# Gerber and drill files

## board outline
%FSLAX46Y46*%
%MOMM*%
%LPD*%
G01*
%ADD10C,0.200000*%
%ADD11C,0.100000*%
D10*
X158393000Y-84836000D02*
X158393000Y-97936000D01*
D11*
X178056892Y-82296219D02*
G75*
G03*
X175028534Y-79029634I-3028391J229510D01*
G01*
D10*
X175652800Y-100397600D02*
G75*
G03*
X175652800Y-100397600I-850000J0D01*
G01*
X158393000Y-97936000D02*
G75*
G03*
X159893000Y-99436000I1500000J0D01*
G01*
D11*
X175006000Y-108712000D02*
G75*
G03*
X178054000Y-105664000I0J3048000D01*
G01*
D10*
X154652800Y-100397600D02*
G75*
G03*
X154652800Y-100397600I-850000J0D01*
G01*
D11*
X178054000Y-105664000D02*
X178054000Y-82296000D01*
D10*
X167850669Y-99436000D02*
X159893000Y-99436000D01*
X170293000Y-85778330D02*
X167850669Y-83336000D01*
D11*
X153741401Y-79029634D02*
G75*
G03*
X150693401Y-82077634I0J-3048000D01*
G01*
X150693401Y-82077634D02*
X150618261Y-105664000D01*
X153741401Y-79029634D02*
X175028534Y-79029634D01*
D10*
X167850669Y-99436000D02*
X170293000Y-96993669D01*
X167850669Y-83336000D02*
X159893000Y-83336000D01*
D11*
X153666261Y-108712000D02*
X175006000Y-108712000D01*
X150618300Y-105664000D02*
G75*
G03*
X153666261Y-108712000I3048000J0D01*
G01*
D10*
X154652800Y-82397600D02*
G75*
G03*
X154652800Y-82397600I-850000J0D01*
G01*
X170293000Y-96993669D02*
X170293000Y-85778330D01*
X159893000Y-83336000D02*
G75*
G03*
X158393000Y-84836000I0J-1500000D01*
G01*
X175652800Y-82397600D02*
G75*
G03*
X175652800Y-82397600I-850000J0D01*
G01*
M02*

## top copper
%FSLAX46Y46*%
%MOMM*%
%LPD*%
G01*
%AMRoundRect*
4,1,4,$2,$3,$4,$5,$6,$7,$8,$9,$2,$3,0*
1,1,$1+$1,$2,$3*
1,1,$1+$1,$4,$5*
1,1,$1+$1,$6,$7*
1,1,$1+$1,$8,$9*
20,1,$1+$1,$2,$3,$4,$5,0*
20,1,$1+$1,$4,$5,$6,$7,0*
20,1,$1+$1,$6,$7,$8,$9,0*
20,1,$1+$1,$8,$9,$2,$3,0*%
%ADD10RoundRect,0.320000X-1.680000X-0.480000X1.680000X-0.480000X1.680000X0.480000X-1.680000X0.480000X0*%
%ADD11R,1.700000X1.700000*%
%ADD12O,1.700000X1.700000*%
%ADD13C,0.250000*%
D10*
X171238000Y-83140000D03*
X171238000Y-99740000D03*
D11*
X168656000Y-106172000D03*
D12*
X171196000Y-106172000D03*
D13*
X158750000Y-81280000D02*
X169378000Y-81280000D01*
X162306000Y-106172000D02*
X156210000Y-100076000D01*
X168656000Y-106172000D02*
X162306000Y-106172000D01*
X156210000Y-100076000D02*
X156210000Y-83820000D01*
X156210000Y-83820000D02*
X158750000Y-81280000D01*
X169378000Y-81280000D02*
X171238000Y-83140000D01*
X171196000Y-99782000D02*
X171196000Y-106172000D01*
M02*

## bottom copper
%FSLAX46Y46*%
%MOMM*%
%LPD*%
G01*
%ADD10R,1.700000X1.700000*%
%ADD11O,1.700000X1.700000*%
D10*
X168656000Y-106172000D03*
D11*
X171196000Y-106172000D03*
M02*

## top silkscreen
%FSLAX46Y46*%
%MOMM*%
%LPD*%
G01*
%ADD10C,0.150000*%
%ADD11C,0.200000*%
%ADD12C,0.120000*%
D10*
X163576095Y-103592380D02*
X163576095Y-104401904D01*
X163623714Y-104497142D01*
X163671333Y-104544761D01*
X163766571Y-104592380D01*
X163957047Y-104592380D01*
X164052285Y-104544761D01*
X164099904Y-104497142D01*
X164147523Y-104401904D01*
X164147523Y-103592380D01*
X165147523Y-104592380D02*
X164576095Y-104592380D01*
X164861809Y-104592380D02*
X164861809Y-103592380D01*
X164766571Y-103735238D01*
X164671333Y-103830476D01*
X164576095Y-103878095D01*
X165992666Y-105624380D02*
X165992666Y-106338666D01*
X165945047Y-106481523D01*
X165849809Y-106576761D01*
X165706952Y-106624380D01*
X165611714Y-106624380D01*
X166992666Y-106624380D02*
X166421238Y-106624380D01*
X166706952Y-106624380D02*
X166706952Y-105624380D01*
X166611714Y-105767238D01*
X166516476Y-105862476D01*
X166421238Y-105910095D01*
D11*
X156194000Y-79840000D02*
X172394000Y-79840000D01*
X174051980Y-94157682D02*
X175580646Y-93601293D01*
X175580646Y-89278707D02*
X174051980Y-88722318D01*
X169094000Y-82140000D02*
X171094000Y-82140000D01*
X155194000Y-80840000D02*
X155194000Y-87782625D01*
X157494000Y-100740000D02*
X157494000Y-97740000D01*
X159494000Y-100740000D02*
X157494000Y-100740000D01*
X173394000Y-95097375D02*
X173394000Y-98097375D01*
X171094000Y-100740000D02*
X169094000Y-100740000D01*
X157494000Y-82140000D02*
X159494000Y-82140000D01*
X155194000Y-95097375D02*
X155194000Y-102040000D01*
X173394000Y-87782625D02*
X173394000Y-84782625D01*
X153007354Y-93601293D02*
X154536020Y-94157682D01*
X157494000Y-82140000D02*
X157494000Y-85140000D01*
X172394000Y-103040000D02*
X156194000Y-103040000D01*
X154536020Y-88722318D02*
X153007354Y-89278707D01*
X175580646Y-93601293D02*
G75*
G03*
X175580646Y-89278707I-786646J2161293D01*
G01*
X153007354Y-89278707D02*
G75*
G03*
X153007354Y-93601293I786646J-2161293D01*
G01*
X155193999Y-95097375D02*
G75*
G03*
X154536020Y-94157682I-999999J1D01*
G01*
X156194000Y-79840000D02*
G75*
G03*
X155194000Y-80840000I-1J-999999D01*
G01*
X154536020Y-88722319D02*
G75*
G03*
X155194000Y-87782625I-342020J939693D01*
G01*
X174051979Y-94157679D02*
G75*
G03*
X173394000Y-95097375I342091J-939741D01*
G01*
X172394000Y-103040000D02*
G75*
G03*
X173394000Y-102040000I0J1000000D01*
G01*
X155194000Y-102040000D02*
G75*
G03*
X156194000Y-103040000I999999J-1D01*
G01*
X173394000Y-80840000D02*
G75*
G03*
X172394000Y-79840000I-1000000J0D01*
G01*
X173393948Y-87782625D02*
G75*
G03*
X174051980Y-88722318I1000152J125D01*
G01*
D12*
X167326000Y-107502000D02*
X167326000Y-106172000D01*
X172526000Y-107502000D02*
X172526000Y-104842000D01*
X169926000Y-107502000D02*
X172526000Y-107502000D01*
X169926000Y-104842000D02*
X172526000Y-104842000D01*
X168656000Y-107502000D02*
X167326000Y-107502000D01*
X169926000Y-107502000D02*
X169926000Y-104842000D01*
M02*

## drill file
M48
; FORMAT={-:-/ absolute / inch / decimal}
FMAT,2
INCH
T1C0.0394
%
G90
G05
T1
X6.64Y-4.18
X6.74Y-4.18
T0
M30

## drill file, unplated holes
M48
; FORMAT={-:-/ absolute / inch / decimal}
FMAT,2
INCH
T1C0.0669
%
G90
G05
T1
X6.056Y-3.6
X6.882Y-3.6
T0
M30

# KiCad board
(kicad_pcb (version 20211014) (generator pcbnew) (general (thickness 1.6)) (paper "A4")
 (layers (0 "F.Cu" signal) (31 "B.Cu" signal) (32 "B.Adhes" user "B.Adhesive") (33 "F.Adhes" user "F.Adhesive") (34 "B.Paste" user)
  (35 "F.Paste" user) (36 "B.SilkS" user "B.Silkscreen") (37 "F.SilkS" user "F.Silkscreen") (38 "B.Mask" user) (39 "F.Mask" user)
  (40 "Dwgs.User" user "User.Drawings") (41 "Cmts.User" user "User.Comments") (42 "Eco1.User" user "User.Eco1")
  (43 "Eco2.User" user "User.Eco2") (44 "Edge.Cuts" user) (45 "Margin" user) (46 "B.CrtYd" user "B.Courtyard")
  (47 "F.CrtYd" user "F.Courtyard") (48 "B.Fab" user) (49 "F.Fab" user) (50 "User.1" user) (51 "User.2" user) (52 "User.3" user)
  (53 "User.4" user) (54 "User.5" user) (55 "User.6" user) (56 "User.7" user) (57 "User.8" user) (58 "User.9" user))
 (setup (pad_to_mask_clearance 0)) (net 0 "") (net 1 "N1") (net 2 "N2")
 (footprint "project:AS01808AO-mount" (layer "F.Cu") (at 164.338 91.44)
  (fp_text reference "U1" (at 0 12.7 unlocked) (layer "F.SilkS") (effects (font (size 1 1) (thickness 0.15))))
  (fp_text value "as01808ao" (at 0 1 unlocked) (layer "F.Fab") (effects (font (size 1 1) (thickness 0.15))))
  (fp_line (start -8.144 -11.6) (end 8.056 -11.6) (layer "F.SilkS") (width 0.2))
  (fp_line (start 9.71398 2.717682) (end 11.242646 2.161293) (layer "F.SilkS") (width 0.2))
  (fp_line (start 11.242646 -2.161293) (end 9.71398 -2.717682) (layer "F.SilkS") (width 0.2))
  (fp_line (start 4.756 -9.3) (end 6.756 -9.3) (layer "F.SilkS") (width 0.2))
  (fp_line (start -9.144 -10.6) (end -9.144 -3.657375) (layer "F.SilkS") (width 0.2))
  (fp_line (start -6.844 9.3) (end -6.844 6.3) (layer "F.SilkS") (width 0.2))
  (fp_line (start -4.844 9.3) (end -6.844 9.3) (layer "F.SilkS") (width 0.2))
  (fp_line (start 9.056 3.657375) (end 9.056 6.657375) (layer "F.SilkS") (width 0.2))
  (fp_line (start 6.756 9.3) (end 4.756 9.3) (layer "F.SilkS") (width 0.2))
  (fp_line (start -6.844 -9.3) (end -4.844 -9.3) (layer "F.SilkS") (width 0.2))
  (fp_line (start -9.144 3.657375) (end -9.144 10.6) (layer "F.SilkS") (width 0.2))
  (fp_line (start 9.056 -3.657375) (end 9.056 -6.657375) (layer "F.SilkS") (width 0.2))
  (fp_line (start -11.330646 2.161293) (end -9.80198 2.717682) (layer "F.SilkS") (width 0.2))
  (fp_line (start -6.844 -9.3) (end -6.844 -6.3) (layer "F.SilkS") (width 0.2))
  (fp_line (start 8.056 11.6) (end -8.144 11.6) (layer "F.SilkS") (width 0.2))
  (fp_line (start -9.80198 -2.717682) (end -11.330646 -2.161293) (layer "F.SilkS") (width 0.2))
  (fp_arc (start 11.242646 -2.161293) (mid 12.756 0) (end 11.242646 2.161293) (layer "F.SilkS") (width 0.2))
  (fp_arc (start -11.330646 2.161293) (mid -12.844 0) (end -11.330646 -2.161293) (layer "F.SilkS") (width 0.2))
  (fp_arc (start -9.80198 2.717682) (mid -9.324848 3.083798) (end -9.144 3.657375) (layer "F.SilkS") (width 0.2))
  (fp_arc (start -9.144 -10.6) (mid -8.851107 -11.307107) (end -8.144 -11.6) (layer "F.SilkS") (width 0.2))
  (fp_arc (start -9.144 -3.657375) (mid -9.324848 -3.083798) (end -9.80198 -2.717682) (layer "F.SilkS") (width 0.2))
  (fp_arc (start 9.056 3.657375) (mid 9.236859 3.083806) (end 9.71398 2.717682) (layer "F.SilkS") (width 0.2))
  (fp_arc (start 9.056 10.6) (mid 8.763107 11.307107) (end 8.056 11.6) (layer "F.SilkS") (width 0.2))
  (fp_arc (start -8.144 11.6) (mid -8.851107 11.307107) (end -9.144 10.6) (layer "F.SilkS") (width 0.2))
  (fp_arc (start 8.056 -11.6) (mid 8.763107 -11.307107) (end 9.056 -10.6) (layer "F.SilkS") (width 0.2))
  (fp_arc (start 9.71398 -2.717682) (mid 9.236845 -3.083806) (end 9.056 -3.657375) (layer "F.SilkS") (width 0.2))
  (pad "" np_thru_hole circle (at 10.4648 0) (size 1.7 1.7) (drill 1.7) (layers F&B.Cu *.Mask))
  (pad "" np_thru_hole circle (at -10.5156 0) (size 1.7 1.7) (drill 1.7) (layers F&B.Cu *.Mask))
  (pad "1" smd roundrect (at 6.9 -8.3) (size 4 1.6) (layers "F.Cu" "F.Paste" "F.Mask") (roundrect_rratio 0.2) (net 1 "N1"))
  (pad "2" smd roundrect (at 6.9 8.3) (size 4 1.6) (layers "F.Cu" "F.Paste" "F.Mask") (roundrect_rratio 0.2) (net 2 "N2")))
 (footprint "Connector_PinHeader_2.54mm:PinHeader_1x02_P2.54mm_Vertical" (layer "F.Cu") (at 168.656 106.172 90)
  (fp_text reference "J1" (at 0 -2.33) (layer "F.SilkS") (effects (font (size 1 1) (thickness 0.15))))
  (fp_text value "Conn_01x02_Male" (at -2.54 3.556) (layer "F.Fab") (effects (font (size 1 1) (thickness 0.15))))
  (fp_line (start -1.33 -1.33) (end 0 -1.33) (layer "F.SilkS") (width 0.12))
  (fp_line (start -1.33 3.87) (end 1.33 3.87) (layer "F.SilkS") (width 0.12))
  (fp_line (start -1.33 1.27) (end -1.33 3.87) (layer "F.SilkS") (width 0.12))
  (fp_line (start 1.33 1.27) (end 1.33 3.87) (layer "F.SilkS") (width 0.12))
  (fp_line (start -1.33 0) (end -1.33 -1.33) (layer "F.SilkS") (width 0.12))
  (fp_line (start -1.33 1.27) (end 1.33 1.27) (layer "F.SilkS") (width 0.12))
  (pad "1" thru_hole rect (at 0 0 90) (size 1.7 1.7) (drill 1) (layers *.Cu *.Mask) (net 1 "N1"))
  (pad "2" thru_hole oval (at 0 2.54 90) (size 1.7 1.7) (drill 1) (layers *.Cu *.Mask) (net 2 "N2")))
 (gr_line (start 158.393 84.836) (end 158.393 97.936) (layer "Edge.Cuts") (width 0.2))
 (gr_arc (start 175.028534 79.029634) (mid 177.255715 80.001923) (end 178.054 82.296) (layer "Edge.Cuts") (width 0.1))
 (gr_circle (center 174.8028 100.3976) (end 175.6528 100.3976) (layer "Edge.Cuts") (width 0.2) (fill none))
 (gr_arc (start 159.893 99.436) (mid 158.83234 98.99666) (end 158.393 97.936) (layer "Edge.Cuts") (width 0.2))
 (gr_arc (start 178.054 105.664) (mid 177.161261 107.819261) (end 175.006 108.712) (layer "Edge.Cuts") (width 0.1))
 (gr_circle (center 153.8028 100.3976) (end 154.6528 100.3976) (layer "Edge.Cuts") (width 0.2) (fill none))
 (gr_line (start 178.054 105.664) (end 178.054 82.296) (layer "Edge.Cuts") (width 0.1))
 (gr_line (start 167.850669 99.436) (end 159.893 99.436) (layer "Edge.Cuts") (width 0.2))
 (gr_line (start 170.293 85.77833) (end 167.850669 83.336) (layer "Edge.Cuts") (width 0.2))
 (gr_arc (start 150.693401 82.077634) (mid 151.58614 79.922373) (end 153.741401 79.029634) (layer "Edge.Cuts") (width 0.1))
 (gr_line (start 150.693401 82.077634) (end 150.618261 105.664) (layer "Edge.Cuts") (width 0.1))
 (gr_line (start 153.741401 79.029634) (end 175.028534 79.029634) (layer "Edge.Cuts") (width 0.1))
 (gr_line (start 167.850669 99.436) (end 170.293 96.993669) (layer "Edge.Cuts") (width 0.2))
 (gr_line (start 167.850669 83.336) (end 159.893 83.336) (layer "Edge.Cuts") (width 0.2))
 (gr_line (start 153.666261 108.712) (end 175.006 108.712) (layer "Edge.Cuts") (width 0.1))
 (gr_arc (start 153.666261 108.712) (mid 151.511 107.819261) (end 150.618261 105.664) (layer "Edge.Cuts") (width 0.1))
 (gr_circle (center 153.8028 82.3976) (end 154.6528 82.3976) (layer "Edge.Cuts") (width 0.2) (fill none))
 (gr_line (start 170.293 96.993669) (end 170.293 85.77833) (layer "Edge.Cuts") (width 0.2))
 (gr_arc (start 158.393 84.836) (mid 158.83234 83.77534) (end 159.893 83.336) (layer "Edge.Cuts") (width 0.2))
 (gr_circle (center 174.8028 82.3976) (end 175.6528 82.3976) (layer "Edge.Cuts") (width 0.2) (fill none))
 (segment (start 158.75 81.28) (end 169.378 81.28) (width 0.25) (layer "F.Cu") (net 1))
 (segment (start 162.306 106.172) (end 156.21 100.076) (width 0.25) (layer "F.Cu") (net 1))
 (segment (start 168.656 106.172) (end 162.306 106.172) (width 0.25) (layer "F.Cu") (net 1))
 (segment (start 156.21 100.076) (end 156.21 83.82) (width 0.25) (layer "F.Cu") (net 1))
 (segment (start 156.21 83.82) (end 158.75 81.28) (width 0.25) (layer "F.Cu") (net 1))
 (segment (start 169.378 81.28) (end 171.238 83.14) (width 0.25) (layer "F.Cu") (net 1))
 (segment (start 171.196 99.782) (end 171.196 106.172) (width 0.25) (layer "F.Cu") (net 2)))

